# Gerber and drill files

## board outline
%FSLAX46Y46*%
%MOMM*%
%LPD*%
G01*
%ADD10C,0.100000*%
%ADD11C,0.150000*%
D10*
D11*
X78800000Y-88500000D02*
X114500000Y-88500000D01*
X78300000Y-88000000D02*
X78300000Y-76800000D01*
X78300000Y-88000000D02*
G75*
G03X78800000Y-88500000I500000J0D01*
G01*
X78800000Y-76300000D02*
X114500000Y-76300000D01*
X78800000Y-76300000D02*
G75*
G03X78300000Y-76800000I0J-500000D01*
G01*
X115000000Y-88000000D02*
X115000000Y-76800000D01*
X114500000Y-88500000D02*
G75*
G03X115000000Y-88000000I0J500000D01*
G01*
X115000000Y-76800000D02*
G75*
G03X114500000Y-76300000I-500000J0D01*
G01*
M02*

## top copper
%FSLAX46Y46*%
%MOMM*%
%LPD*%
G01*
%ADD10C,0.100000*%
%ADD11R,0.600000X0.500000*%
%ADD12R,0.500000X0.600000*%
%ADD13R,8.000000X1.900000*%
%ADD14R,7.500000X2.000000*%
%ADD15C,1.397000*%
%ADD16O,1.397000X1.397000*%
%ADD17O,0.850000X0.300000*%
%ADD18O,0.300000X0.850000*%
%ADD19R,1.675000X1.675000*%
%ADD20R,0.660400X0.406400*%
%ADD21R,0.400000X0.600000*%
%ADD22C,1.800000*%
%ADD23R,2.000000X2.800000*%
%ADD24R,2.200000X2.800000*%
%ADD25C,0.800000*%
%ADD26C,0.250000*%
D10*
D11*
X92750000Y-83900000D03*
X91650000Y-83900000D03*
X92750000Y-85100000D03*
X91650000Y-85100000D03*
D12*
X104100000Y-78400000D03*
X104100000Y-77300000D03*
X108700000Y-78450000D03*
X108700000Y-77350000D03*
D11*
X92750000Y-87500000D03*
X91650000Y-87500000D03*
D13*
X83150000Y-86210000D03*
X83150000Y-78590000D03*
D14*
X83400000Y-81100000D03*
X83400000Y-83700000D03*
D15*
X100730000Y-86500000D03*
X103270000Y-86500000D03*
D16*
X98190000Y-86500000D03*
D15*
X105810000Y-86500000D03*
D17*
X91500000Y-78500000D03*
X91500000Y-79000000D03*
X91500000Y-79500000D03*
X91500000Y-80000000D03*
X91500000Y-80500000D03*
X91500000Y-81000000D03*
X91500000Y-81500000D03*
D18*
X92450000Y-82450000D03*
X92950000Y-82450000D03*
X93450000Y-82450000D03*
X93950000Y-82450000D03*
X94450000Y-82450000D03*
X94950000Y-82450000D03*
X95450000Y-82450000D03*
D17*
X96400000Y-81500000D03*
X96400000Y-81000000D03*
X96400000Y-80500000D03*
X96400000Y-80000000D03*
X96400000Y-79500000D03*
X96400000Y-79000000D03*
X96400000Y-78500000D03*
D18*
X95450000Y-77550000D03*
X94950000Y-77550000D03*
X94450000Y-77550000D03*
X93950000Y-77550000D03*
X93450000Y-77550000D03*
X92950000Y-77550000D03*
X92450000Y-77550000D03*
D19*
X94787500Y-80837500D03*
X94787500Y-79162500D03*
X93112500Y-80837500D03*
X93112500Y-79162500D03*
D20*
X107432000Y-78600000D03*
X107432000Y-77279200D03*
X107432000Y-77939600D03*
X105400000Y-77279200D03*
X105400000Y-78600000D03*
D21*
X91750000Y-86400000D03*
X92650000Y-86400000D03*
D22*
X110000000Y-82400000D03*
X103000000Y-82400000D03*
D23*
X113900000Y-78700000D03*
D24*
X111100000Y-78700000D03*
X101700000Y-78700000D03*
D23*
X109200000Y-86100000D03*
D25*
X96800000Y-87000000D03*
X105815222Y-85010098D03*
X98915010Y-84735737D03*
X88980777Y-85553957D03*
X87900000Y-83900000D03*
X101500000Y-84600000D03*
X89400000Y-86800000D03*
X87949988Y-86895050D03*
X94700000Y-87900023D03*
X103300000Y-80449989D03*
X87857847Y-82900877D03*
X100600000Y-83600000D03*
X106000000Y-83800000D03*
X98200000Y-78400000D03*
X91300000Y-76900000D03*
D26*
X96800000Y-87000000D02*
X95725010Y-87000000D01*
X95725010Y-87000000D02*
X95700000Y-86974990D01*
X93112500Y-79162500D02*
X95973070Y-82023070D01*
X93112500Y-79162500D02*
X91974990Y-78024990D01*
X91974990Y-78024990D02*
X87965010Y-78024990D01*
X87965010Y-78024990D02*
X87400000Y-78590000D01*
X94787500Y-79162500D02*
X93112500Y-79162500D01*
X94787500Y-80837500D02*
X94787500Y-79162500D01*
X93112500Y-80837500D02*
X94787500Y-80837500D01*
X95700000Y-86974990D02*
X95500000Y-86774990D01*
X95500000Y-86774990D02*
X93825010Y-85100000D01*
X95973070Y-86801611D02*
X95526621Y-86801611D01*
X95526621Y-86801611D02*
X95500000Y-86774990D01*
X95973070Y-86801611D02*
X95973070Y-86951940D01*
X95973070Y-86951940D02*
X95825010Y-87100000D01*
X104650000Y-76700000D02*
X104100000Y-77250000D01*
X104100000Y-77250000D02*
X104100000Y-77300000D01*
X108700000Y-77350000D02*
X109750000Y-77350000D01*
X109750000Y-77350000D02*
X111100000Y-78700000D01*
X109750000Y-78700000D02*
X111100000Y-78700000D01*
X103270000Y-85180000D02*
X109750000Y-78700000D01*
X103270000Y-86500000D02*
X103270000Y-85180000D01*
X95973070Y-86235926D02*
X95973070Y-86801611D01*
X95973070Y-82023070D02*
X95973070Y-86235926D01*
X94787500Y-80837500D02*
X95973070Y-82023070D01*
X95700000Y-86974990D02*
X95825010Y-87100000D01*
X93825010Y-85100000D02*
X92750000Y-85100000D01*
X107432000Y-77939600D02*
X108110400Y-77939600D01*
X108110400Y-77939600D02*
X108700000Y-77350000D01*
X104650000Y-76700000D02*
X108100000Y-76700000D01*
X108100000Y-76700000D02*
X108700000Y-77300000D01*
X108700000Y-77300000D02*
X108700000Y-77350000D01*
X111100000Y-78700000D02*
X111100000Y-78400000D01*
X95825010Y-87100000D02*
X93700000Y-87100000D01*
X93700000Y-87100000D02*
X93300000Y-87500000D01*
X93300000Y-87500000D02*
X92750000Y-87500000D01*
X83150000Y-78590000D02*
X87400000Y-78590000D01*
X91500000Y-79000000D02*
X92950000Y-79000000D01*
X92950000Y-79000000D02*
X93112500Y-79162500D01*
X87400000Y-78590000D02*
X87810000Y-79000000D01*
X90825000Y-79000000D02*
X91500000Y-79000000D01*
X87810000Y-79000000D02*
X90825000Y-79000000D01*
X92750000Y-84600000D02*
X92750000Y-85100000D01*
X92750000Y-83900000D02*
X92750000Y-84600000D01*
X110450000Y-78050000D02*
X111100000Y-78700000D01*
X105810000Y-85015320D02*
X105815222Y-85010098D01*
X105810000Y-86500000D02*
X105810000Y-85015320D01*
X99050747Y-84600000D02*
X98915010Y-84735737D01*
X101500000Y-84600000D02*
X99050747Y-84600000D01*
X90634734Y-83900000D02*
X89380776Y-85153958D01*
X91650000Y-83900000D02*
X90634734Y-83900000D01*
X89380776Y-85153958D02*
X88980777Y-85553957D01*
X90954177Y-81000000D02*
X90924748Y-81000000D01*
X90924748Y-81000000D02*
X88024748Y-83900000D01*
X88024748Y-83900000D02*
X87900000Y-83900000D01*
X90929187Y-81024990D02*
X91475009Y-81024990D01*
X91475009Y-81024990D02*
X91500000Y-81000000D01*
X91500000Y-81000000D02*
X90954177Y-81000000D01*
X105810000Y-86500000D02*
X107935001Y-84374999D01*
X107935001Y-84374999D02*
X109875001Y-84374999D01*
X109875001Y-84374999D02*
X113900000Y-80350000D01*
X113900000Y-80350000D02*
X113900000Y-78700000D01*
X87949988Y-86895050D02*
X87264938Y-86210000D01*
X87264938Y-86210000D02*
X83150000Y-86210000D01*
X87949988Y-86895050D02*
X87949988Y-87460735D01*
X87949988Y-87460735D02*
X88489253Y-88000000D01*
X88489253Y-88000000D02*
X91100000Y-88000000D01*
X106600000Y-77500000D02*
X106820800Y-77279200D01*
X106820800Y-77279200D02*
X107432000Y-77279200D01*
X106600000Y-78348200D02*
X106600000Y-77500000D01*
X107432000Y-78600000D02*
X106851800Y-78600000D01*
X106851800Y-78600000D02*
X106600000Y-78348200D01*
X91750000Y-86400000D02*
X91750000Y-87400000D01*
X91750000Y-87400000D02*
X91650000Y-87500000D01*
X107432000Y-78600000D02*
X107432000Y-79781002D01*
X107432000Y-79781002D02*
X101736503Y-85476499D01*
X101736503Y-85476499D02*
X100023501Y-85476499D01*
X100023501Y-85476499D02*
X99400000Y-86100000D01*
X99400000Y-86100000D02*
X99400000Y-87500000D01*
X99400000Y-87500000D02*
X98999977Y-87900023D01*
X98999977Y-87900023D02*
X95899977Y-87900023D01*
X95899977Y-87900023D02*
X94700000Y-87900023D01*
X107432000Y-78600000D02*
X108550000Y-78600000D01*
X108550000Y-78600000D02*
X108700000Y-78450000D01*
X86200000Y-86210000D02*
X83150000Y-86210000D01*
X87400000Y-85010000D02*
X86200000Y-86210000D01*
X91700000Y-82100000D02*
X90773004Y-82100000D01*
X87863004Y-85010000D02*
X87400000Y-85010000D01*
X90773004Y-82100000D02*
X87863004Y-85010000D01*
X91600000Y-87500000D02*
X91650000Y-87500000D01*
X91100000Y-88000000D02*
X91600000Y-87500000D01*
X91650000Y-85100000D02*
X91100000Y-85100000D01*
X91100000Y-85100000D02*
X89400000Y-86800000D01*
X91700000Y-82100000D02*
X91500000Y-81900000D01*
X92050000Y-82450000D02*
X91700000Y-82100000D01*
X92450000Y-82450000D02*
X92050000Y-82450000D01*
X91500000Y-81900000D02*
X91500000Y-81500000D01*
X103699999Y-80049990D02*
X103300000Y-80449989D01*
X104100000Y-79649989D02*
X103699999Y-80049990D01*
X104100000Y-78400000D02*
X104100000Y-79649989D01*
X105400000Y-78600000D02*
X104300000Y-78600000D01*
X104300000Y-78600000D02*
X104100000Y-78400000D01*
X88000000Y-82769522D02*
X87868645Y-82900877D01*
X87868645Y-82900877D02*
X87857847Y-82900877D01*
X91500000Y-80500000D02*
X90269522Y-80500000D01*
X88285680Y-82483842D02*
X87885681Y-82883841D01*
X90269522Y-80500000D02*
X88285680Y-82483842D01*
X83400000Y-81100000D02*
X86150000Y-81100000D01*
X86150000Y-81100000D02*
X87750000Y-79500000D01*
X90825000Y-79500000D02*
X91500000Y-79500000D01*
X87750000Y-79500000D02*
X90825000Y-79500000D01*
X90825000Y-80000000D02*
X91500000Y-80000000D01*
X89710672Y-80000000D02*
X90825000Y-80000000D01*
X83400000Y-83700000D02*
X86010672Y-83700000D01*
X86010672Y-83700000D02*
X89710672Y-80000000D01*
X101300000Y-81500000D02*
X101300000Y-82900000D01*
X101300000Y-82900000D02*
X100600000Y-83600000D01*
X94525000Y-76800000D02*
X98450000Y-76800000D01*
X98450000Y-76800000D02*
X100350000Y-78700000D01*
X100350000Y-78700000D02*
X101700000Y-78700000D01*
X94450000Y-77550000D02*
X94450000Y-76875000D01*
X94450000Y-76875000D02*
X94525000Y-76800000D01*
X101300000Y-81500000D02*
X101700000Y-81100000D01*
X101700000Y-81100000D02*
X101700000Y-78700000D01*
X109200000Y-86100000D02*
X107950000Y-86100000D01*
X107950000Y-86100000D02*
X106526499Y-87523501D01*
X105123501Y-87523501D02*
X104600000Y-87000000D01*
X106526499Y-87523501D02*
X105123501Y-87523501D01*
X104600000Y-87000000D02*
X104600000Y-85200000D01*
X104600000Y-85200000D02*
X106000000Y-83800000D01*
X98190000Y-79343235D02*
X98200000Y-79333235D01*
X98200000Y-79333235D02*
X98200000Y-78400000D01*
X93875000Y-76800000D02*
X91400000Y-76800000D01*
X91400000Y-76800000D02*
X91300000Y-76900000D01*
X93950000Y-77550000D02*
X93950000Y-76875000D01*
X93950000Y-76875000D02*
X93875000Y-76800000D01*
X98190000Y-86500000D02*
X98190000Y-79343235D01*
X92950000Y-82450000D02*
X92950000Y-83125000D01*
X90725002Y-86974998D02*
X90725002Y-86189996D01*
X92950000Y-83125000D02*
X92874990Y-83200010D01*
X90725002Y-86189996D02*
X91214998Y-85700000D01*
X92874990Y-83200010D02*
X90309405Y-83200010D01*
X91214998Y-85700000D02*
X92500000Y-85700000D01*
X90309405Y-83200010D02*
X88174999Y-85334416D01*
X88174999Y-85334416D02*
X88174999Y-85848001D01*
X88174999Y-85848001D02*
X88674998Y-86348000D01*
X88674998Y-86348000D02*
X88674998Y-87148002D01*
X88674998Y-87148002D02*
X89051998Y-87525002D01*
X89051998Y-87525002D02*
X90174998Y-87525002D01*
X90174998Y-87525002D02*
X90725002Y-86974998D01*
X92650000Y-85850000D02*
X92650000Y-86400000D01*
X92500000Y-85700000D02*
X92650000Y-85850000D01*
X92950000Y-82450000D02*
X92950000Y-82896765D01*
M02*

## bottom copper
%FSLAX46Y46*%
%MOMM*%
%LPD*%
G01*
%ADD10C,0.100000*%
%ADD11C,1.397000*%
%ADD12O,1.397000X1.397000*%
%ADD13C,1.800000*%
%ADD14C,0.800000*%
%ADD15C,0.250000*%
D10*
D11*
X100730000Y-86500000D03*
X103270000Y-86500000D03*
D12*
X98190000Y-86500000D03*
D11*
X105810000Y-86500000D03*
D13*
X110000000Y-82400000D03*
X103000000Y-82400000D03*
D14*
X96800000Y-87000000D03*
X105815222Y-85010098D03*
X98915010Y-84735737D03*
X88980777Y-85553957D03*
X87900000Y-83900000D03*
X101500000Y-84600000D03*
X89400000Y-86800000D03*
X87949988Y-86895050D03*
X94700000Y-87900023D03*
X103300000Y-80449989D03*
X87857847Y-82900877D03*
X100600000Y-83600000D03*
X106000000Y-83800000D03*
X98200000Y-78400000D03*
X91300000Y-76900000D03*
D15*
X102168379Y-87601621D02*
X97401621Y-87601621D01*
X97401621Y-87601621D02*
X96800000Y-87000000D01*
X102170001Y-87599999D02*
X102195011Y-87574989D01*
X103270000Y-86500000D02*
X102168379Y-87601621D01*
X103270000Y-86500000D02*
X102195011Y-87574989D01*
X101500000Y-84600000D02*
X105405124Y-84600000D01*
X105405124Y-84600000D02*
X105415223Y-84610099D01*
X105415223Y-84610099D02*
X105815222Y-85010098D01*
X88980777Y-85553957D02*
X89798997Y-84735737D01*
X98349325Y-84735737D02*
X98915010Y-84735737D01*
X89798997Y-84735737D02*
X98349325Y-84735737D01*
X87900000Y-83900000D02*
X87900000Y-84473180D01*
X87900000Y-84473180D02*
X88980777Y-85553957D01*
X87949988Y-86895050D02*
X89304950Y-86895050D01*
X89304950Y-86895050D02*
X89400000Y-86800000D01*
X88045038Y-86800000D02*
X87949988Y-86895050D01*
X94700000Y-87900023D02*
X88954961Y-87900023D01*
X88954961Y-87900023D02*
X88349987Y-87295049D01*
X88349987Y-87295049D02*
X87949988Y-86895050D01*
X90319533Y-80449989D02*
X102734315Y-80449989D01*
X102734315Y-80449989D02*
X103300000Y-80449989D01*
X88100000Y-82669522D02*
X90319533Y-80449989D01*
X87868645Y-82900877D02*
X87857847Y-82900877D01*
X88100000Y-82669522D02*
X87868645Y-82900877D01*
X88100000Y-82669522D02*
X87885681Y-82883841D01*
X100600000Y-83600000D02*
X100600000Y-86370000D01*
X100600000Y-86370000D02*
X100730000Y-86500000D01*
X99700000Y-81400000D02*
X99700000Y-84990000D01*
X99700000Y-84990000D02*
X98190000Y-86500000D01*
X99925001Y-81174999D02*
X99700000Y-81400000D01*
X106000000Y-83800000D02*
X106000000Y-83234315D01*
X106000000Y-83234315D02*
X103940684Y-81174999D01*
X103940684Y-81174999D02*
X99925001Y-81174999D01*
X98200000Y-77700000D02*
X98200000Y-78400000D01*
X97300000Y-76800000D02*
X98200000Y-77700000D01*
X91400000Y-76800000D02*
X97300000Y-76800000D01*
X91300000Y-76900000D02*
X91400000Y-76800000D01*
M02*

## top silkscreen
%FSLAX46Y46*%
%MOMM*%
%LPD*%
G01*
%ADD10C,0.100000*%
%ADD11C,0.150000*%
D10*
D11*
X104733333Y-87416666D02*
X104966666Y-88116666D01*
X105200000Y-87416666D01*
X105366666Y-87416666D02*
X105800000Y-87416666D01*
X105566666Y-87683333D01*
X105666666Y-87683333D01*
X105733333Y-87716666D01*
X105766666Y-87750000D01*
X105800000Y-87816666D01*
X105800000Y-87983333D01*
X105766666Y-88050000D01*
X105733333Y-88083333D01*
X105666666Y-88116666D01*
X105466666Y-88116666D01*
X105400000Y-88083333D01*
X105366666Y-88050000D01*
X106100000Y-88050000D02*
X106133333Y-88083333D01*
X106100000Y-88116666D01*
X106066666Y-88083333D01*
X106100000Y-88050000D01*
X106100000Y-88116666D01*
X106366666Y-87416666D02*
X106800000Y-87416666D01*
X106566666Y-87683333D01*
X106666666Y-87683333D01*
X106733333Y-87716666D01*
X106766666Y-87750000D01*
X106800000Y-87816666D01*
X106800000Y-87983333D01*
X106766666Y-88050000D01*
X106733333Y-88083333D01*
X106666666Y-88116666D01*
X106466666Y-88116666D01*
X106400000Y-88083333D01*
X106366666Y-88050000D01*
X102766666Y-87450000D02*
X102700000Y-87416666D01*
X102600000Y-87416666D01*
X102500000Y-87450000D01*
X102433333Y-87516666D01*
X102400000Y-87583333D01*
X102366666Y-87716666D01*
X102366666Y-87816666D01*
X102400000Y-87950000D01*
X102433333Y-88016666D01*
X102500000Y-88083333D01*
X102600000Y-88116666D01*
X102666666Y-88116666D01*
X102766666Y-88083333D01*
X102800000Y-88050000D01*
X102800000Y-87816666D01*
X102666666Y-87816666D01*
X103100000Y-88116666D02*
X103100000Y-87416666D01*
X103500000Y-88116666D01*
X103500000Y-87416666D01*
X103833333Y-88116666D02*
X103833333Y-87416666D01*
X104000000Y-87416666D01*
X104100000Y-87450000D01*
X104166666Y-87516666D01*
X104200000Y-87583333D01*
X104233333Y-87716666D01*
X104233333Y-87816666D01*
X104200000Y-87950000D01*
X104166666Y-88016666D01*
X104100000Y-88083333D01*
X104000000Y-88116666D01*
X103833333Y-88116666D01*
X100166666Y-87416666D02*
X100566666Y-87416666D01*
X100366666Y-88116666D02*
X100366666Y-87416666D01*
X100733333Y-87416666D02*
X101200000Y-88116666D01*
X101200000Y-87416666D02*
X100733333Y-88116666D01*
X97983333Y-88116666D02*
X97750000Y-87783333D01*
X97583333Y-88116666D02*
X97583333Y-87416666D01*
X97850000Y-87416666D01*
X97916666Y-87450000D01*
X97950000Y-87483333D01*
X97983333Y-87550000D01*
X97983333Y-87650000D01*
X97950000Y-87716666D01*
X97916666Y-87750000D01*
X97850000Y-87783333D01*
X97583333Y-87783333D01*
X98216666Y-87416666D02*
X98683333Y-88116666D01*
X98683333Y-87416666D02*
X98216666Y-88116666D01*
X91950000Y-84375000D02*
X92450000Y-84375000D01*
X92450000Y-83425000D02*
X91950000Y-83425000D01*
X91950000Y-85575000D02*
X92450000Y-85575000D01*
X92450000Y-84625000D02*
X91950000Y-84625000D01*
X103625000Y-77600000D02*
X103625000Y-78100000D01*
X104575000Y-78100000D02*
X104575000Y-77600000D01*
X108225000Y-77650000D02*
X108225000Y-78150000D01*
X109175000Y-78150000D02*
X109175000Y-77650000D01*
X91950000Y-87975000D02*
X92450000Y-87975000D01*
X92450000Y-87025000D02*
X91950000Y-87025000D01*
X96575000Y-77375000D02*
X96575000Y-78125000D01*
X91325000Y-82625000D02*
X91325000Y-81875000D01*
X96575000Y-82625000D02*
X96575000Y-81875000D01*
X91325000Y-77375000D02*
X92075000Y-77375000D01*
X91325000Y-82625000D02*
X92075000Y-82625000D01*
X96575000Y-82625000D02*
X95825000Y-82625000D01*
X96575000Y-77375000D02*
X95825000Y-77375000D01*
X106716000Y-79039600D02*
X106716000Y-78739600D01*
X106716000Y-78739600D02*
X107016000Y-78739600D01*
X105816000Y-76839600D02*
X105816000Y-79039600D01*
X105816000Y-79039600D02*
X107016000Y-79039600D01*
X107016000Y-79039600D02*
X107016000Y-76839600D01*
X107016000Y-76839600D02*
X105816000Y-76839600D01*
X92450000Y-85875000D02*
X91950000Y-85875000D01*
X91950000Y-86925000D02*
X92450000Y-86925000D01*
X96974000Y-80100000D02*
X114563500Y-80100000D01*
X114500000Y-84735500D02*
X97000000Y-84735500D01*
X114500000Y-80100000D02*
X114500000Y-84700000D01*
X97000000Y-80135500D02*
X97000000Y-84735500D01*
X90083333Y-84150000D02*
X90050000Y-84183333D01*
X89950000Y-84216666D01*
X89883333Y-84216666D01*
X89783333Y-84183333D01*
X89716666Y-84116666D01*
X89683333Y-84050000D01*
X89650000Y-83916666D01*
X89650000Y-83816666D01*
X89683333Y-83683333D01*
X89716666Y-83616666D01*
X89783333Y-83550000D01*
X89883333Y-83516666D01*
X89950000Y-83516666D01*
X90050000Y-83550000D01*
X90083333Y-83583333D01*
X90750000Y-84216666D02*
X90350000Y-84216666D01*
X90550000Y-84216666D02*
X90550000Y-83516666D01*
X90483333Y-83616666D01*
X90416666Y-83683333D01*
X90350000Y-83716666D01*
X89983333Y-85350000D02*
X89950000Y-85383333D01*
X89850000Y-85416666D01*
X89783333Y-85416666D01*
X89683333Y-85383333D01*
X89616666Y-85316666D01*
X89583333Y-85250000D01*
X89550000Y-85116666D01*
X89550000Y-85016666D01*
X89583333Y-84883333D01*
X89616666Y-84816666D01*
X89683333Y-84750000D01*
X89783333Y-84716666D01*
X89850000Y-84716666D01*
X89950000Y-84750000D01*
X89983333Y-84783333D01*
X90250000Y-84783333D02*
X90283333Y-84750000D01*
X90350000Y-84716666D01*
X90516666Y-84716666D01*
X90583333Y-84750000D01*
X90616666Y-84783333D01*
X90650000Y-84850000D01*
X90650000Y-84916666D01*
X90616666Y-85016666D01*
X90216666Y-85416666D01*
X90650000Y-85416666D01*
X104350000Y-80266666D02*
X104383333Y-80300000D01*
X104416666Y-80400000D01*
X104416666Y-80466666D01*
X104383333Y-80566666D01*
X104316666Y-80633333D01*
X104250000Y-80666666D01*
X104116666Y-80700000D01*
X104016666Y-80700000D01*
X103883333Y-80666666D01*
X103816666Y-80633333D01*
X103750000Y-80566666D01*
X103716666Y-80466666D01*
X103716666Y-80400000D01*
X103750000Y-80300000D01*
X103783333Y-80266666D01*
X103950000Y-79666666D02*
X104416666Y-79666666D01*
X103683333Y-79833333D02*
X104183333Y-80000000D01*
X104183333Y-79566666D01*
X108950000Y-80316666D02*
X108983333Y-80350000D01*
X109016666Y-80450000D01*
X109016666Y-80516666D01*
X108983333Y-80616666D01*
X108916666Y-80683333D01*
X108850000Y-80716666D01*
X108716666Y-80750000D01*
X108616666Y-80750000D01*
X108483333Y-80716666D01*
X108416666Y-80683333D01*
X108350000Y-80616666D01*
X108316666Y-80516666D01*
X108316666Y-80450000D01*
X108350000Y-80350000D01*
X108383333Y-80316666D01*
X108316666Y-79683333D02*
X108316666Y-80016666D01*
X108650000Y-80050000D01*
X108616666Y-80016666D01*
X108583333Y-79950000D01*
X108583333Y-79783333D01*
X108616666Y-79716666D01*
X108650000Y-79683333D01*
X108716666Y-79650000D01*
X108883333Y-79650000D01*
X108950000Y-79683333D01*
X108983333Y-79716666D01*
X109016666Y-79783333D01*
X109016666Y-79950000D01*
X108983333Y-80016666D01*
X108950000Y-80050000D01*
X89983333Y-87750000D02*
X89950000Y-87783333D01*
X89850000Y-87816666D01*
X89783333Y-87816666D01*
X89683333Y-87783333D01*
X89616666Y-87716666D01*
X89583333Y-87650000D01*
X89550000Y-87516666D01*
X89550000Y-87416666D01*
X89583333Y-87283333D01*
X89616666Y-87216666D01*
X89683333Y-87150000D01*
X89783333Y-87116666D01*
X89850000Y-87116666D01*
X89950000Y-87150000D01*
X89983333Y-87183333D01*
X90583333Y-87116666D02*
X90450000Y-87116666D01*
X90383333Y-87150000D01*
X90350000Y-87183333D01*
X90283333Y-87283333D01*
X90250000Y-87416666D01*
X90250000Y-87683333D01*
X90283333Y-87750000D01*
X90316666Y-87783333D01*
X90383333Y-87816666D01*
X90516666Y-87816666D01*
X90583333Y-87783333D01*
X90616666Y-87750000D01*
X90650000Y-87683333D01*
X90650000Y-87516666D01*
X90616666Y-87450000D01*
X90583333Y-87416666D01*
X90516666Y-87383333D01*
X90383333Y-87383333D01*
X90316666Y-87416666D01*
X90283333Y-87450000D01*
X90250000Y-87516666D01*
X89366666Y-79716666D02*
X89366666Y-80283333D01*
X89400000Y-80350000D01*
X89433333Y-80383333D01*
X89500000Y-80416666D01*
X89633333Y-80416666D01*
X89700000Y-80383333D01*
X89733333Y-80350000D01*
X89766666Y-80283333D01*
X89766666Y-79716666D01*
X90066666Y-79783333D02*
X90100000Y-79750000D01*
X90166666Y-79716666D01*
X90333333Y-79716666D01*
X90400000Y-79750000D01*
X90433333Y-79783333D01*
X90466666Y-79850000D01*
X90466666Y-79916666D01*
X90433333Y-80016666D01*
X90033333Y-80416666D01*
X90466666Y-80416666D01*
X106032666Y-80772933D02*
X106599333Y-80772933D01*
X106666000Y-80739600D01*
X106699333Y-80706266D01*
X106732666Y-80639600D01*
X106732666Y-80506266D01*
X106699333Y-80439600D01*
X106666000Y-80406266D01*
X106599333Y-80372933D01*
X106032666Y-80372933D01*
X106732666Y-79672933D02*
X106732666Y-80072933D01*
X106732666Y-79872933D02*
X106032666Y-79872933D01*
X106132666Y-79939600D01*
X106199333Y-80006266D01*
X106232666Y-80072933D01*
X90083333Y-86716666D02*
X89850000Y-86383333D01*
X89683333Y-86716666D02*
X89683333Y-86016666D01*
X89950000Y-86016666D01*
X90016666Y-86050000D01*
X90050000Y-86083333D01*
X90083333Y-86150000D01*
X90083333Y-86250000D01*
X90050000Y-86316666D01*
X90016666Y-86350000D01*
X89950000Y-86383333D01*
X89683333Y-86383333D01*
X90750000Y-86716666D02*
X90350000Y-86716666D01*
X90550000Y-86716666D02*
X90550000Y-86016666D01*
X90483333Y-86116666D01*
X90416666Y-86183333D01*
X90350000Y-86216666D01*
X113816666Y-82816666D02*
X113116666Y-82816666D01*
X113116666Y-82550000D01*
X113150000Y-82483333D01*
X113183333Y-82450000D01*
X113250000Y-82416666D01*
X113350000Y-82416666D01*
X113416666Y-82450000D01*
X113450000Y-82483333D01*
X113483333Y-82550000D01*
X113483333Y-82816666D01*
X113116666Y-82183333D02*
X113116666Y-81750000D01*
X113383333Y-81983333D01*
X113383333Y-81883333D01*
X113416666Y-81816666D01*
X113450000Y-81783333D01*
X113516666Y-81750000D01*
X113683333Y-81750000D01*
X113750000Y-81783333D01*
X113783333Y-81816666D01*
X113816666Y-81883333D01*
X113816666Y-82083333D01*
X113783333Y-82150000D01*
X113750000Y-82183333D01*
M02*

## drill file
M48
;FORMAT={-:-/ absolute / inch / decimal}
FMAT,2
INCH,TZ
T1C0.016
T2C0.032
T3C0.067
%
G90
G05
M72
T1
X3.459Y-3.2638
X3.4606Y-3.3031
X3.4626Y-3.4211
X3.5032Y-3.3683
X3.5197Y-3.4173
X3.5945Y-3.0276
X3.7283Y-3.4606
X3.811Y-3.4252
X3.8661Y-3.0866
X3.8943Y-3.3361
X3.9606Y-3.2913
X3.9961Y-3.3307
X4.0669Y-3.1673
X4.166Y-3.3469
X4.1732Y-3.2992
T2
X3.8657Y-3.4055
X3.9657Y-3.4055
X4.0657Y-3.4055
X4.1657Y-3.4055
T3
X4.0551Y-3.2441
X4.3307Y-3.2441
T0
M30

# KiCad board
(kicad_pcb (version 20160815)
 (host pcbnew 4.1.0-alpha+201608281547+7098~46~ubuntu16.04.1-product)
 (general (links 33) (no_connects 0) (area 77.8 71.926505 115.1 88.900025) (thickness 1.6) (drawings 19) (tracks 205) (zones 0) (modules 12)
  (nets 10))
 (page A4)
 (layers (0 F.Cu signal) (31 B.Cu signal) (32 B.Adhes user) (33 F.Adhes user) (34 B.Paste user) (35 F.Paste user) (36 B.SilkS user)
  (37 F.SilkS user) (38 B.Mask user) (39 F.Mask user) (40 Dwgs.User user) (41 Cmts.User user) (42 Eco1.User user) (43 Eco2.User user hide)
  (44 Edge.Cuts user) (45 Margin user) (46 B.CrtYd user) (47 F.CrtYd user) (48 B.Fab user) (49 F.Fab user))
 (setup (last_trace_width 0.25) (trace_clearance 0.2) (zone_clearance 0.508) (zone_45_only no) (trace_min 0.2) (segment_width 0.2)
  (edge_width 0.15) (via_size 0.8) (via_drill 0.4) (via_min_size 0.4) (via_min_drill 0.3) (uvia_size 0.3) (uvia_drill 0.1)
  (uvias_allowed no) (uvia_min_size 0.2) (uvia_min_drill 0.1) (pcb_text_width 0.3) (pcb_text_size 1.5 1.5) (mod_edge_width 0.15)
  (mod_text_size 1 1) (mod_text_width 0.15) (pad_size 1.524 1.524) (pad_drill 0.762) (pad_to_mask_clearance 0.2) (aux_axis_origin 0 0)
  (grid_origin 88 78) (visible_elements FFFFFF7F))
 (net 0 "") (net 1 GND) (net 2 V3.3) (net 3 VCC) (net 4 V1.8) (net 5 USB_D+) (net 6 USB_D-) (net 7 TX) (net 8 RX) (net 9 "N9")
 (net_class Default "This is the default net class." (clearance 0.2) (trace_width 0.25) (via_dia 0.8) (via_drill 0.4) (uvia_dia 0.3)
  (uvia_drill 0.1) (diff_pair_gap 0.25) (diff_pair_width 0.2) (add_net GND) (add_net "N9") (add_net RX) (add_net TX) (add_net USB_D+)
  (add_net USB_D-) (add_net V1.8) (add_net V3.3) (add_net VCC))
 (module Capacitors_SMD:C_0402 (layer F.Cu) (at 92.2 83.9 180)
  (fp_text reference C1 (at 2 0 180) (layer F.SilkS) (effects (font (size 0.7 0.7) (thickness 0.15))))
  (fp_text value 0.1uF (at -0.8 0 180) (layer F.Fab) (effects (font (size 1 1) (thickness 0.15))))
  (fp_line (start 0.25 -0.475) (end -0.25 -0.475) (layer F.SilkS) (width 0.15))
  (fp_line (start -0.25 0.475) (end 0.25 0.475) (layer F.SilkS) (width 0.15))
  (pad 1 smd rect (at -0.55 0 180) (size 0.6 0.5) (layers F.Cu F.Paste F.Mask) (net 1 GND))
  (pad 2 smd rect (at 0.55 0 180) (size 0.6 0.5) (layers F.Cu F.Paste F.Mask) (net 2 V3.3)))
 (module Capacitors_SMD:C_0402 (layer F.Cu) (at 92.2 85.1 180)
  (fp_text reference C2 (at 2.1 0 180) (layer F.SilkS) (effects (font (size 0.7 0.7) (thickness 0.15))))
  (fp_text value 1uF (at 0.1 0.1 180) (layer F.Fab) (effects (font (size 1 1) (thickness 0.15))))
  (fp_line (start 0.25 -0.475) (end -0.25 -0.475) (layer F.SilkS) (width 0.15))
  (fp_line (start -0.25 0.475) (end 0.25 0.475) (layer F.SilkS) (width 0.15))
  (pad 1 smd rect (at -0.55 0 180) (size 0.6 0.5) (layers F.Cu F.Paste F.Mask) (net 1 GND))
  (pad 2 smd rect (at 0.55 0 180) (size 0.6 0.5) (layers F.Cu F.Paste F.Mask) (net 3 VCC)))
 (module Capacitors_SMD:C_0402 (layer F.Cu) (at 104.1 77.85 90)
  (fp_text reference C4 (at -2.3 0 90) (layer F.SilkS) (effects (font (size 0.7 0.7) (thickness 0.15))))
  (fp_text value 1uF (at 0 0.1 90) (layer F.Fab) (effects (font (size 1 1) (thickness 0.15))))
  (fp_line (start 0.25 -0.475) (end -0.25 -0.475) (layer F.SilkS) (width 0.15))
  (fp_line (start -0.25 0.475) (end 0.25 0.475) (layer F.SilkS) (width 0.15))
  (pad 1 smd rect (at -0.55 0 90) (size 0.6 0.5) (layers F.Cu F.Paste F.Mask) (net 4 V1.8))
  (pad 2 smd rect (at 0.55 0 90) (size 0.6 0.5) (layers F.Cu F.Paste F.Mask) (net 1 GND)))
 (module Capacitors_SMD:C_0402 (layer F.Cu) (at 108.7 77.9 90)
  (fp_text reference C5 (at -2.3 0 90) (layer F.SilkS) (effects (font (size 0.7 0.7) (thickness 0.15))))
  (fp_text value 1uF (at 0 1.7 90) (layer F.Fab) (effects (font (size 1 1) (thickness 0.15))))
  (fp_line (start 0.25 -0.475) (end -0.25 -0.475) (layer F.SilkS) (width 0.15))
  (fp_line (start -0.25 0.475) (end 0.25 0.475) (layer F.SilkS) (width 0.15))
  (pad 1 smd rect (at -0.55 0 90) (size 0.6 0.5) (layers F.Cu F.Paste F.Mask) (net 3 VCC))
  (pad 2 smd rect (at 0.55 0 90) (size 0.6 0.5) (layers F.Cu F.Paste F.Mask) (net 1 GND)))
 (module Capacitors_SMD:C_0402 (layer F.Cu) (at 92.2 87.5 180)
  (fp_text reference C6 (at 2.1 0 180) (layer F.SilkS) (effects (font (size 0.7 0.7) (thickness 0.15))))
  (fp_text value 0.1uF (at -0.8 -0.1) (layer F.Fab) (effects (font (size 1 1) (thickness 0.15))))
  (fp_line (start 0.25 -0.475) (end -0.25 -0.475) (layer F.SilkS) (width 0.15))
  (fp_line (start -0.25 0.475) (end 0.25 0.475) (layer F.SilkS) (width 0.15))
  (pad 1 smd rect (at -0.55 0 180) (size 0.6 0.5) (layers F.Cu F.Paste F.Mask) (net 1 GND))
  (pad 2 smd rect (at 0.55 0 180) (size 0.6 0.5) (layers F.Cu F.Paste F.Mask) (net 3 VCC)))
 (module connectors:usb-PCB (layer F.Cu) (at 78.25 82.4 270)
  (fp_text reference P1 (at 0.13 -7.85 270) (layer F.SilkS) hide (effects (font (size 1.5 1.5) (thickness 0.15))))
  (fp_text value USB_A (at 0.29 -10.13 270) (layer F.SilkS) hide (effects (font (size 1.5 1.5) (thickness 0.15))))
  (pad 1 connect rect (at 3.81 -4.9 270) (size 1.9 8) (layers F.Cu F.Mask) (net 3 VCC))
  (pad 4 connect rect (at -3.81 -4.9 270) (size 1.9 8) (layers F.Cu F.Mask) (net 1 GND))
  (pad 3 connect rect (at -1.3 -5.15 270) (size 2 7.5) (layers F.Cu F.Mask) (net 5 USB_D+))
  (pad 2 connect rect (at 1.3 -5.15 270) (size 2 7.5) (layers F.Cu F.Mask) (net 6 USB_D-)))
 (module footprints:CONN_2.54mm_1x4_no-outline (layer F.Cu) (at 102 86.5 180)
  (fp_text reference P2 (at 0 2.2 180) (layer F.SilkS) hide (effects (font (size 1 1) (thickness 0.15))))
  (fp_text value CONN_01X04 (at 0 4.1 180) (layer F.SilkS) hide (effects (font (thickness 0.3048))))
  (pad 2 thru_hole circle (at 1.27 0 180) (size 1.397 1.397) (drill 0.8128) (layers *.Cu *.Mask F.SilkS) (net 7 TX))
  (pad 3 thru_hole circle (at -1.27 0 180) (size 1.397 1.397) (drill 0.8128) (layers *.Cu *.Mask F.SilkS) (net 1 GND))
  (pad 1 thru_hole oval (at 3.81 0 180) (size 1.397 1.397) (drill 0.8128) (layers *.Cu *.Mask F.SilkS) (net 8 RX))
  (pad 4 thru_hole circle (at -3.81 0 180) (size 1.397 1.397) (drill 0.8128) (layers *.Cu *.Mask F.SilkS) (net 2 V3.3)))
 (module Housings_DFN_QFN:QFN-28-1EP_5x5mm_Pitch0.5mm (layer F.Cu) (at 93.95 80)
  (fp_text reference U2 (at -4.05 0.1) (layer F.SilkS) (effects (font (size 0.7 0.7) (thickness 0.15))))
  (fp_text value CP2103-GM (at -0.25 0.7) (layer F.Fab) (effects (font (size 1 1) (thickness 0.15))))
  (fp_line (start 2.625 -2.625) (end 2.625 -1.875) (layer F.SilkS) (width 0.15))
  (fp_line (start -2.625 2.625) (end -2.625 1.875) (layer F.SilkS) (width 0.15))
  (fp_line (start 2.625 2.625) (end 2.625 1.875) (layer F.SilkS) (width 0.15))
  (fp_line (start -2.625 -2.625) (end -1.875 -2.625) (layer F.SilkS) (width 0.15))
  (fp_line (start -2.625 2.625) (end -1.875 2.625) (layer F.SilkS) (width 0.15))
  (fp_line (start 2.625 2.625) (end 1.875 2.625) (layer F.SilkS) (width 0.15))
  (fp_line (start 2.625 -2.625) (end 1.875 -2.625) (layer F.SilkS) (width 0.15))
  (pad 1 smd oval (at -2.45 -1.5) (size 0.85 0.3) (layers F.Cu F.Paste F.Mask))
  (pad 2 smd oval (at -2.45 -1) (size 0.85 0.3) (layers F.Cu F.Paste F.Mask) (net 1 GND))
  (pad 3 smd oval (at -2.45 -0.5) (size 0.85 0.3) (layers F.Cu F.Paste F.Mask) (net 5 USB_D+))
  (pad 4 smd oval (at -2.45 0) (size 0.85 0.3) (layers F.Cu F.Paste F.Mask) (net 6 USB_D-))
  (pad 5 smd oval (at -2.45 0.5) (size 0.85 0.3) (layers F.Cu F.Paste F.Mask) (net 4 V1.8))
  (pad 6 smd oval (at -2.45 1) (size 0.85 0.3) (layers F.Cu F.Paste F.Mask) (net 2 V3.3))
  (pad 7 smd oval (at -2.45 1.5) (size 0.85 0.3) (layers F.Cu F.Paste F.Mask) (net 3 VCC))
  (pad 8 smd oval (at -1.5 2.45 90) (size 0.85 0.3) (layers F.Cu F.Paste F.Mask) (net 3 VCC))
  (pad 9 smd oval (at -1 2.45 90) (size 0.85 0.3) (layers F.Cu F.Paste F.Mask) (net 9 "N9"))
  (pad 10 smd oval (at -0.5 2.45 90) (size 0.85 0.3) (layers F.Cu F.Paste F.Mask))
  (pad 11 smd oval (at 0 2.45 90) (size 0.85 0.3) (layers F.Cu F.Paste F.Mask))
  (pad 12 smd oval (at 0.5 2.45 90) (size 0.85 0.3) (layers F.Cu F.Paste F.Mask))
  (pad 13 smd oval (at 1 2.45 90) (size 0.85 0.3) (layers F.Cu F.Paste F.Mask))
  (pad 14 smd oval (at 1.5 2.45 90) (size 0.85 0.3) (layers F.Cu F.Paste F.Mask))
  (pad 15 smd oval (at 2.45 1.5) (size 0.85 0.3) (layers F.Cu F.Paste F.Mask))
  (pad 16 smd oval (at 2.45 1) (size 0.85 0.3) (layers F.Cu F.Paste F.Mask))
  (pad 17 smd oval (at 2.45 0.5) (size 0.85 0.3) (layers F.Cu F.Paste F.Mask))
  (pad 18 smd oval (at 2.45 0) (size 0.85 0.3) (layers F.Cu F.Paste F.Mask))
  (pad 19 smd oval (at 2.45 -0.5) (size 0.85 0.3) (layers F.Cu F.Paste F.Mask))
  (pad 20 smd oval (at 2.45 -1) (size 0.85 0.3) (layers F.Cu F.Paste F.Mask))
  (pad 21 smd oval (at 2.45 -1.5) (size 0.85 0.3) (layers F.Cu F.Paste F.Mask))
  (pad 22 smd oval (at 1.5 -2.45 90) (size 0.85 0.3) (layers F.Cu F.Paste F.Mask))
  (pad 23 smd oval (at 1 -2.45 90) (size 0.85 0.3) (layers F.Cu F.Paste F.Mask))
  (pad 24 smd oval (at 0.5 -2.45 90) (size 0.85 0.3) (layers F.Cu F.Paste F.Mask) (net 7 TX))
  (pad 25 smd oval (at 0 -2.45 90) (size 0.85 0.3) (layers F.Cu F.Paste F.Mask) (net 8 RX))
  (pad 26 smd oval (at -0.5 -2.45 90) (size 0.85 0.3) (layers F.Cu F.Paste F.Mask))
  (pad 27 smd oval (at -1 -2.45 90) (size 0.85 0.3) (layers F.Cu F.Paste F.Mask))
  (pad 28 smd oval (at -1.5 -2.45 90) (size 0.85 0.3) (layers F.Cu F.Paste F.Mask))
  (pad 29 smd rect (at 0.8375 0.8375) (size 1.675 1.675) (layers F.Cu F.Paste F.Mask) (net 1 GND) (solder_paste_margin_ratio -0.2))
  (pad 29 smd rect (at 0.8375 -0.8375) (size 1.675 1.675) (layers F.Cu F.Paste F.Mask) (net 1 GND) (solder_paste_margin_ratio -0.2))
  (pad 29 smd rect (at -0.8375 0.8375) (size 1.675 1.675) (layers F.Cu F.Paste F.Mask) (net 1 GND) (solder_paste_margin_ratio -0.2))
  (pad 29 smd rect (at -0.8375 -0.8375) (size 1.675 1.675) (layers F.Cu F.Paste F.Mask) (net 1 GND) (solder_paste_margin_ratio -0.2)))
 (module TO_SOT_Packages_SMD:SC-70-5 (layer F.Cu) (at 106.416 77.9396 90)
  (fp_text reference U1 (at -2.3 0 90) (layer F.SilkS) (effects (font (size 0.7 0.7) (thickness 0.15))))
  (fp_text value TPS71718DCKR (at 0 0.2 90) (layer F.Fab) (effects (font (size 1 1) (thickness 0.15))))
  (fp_line (start -1.1 0.3) (end -0.8 0.3) (layer F.SilkS) (width 0.15))
  (fp_line (start -0.8 0.3) (end -0.8 0.6) (layer F.SilkS) (width 0.15))
  (fp_line (start 1.1 -0.6) (end -1.1 -0.6) (layer F.SilkS) (width 0.15))
  (fp_line (start -1.1 -0.6) (end -1.1 0.6) (layer F.SilkS) (width 0.15))
  (fp_line (start -1.1 0.6) (end 1.1 0.6) (layer F.SilkS) (width 0.15))
  (fp_line (start 1.1 0.6) (end 1.1 -0.6) (layer F.SilkS) (width 0.15))
  (pad 1 smd rect (at -0.6604 1.016 90) (size 0.4064 0.6604) (layers F.Cu F.Paste F.Mask) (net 3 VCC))
  (pad 3 smd rect (at 0.6604 1.016 90) (size 0.4064 0.6604) (layers F.Cu F.Paste F.Mask) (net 3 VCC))
  (pad 2 smd rect (at 0 1.016 90) (size 0.4064 0.6604) (layers F.Cu F.Paste F.Mask) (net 1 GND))
  (pad 4 smd rect (at 0.6604 -1.016 90) (size 0.4064 0.6604) (layers F.Cu F.Paste F.Mask))
  (pad 5 smd rect (at -0.6604 -1.016 90) (size 0.4064 0.6604) (layers F.Cu F.Paste F.Mask) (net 4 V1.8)))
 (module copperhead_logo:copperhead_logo (layer B.Cu) (at 94.2 82.1)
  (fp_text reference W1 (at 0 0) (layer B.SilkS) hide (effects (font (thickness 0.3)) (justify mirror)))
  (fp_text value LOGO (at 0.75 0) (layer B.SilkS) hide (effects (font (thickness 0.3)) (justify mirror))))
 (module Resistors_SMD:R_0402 (layer F.Cu) (at 92.2 86.4)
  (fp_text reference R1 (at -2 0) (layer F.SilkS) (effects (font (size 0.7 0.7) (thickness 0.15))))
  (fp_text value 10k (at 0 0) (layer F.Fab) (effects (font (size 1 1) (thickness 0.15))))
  (fp_line (start 0.25 -0.525) (end -0.25 -0.525) (layer F.SilkS) (width 0.15))
  (fp_line (start -0.25 0.525) (end 0.25 0.525) (layer F.SilkS) (width 0.15))
  (pad 1 smd rect (at -0.45 0) (size 0.4 0.6) (layers F.Cu F.Paste F.Mask) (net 3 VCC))
  (pad 2 smd rect (at 0.45 0) (size 0.4 0.6) (layers F.Cu F.Paste F.Mask) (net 9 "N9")))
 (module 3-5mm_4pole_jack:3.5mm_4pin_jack (layer F.Cu) (at 114.5 80.1 270)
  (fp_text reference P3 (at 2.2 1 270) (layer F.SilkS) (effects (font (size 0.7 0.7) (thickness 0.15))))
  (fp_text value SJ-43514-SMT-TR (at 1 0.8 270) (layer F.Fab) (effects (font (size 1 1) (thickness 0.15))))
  (fp_line (start 0 17.526) (end 0 -0.0635) (layer F.SilkS) (width 0.15))
  (fp_line (start 4.6355 0) (end 4.6355 17.5) (layer F.SilkS) (width 0.15))
  (fp_line (start 0 0) (end 4.6 0) (layer F.SilkS) (width 0.15))
  (fp_line (start 0.0355 17.5) (end 4.6355 17.5) (layer F.SilkS) (width 0.15))
  (pad "" np_thru_hole circle (at 2.3 4.5 270) (size 1.8 1.8) (drill 1.7) (layers *.Cu *.Mask))
  (pad "" np_thru_hole circle (at 2.3 11.5 270) (size 1.8 1.8) (drill 1.7) (layers *.Cu *.Mask))
  (pad 1 smd rect (at -1.4 0.6 270) (size 2.8 2) (layers F.Cu F.Paste F.Mask) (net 2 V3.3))
  (pad 4 smd rect (at -1.4 3.4 270) (size 2.8 2.2) (layers F.Cu F.Paste F.Mask) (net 1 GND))
  (pad 2 smd rect (at -1.4 12.8 270) (size 2.8 2.2) (layers F.Cu F.Paste F.Mask) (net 7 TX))
  (pad 3 smd rect (at 6 5.3 270) (size 2.8 2) (layers F.Cu F.Paste F.Mask) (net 8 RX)))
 (gr_line (start 78.8 88.5) (end 114.5 88.5) (layer Edge.Cuts) (width 0.15))
 (gr_line (start 78.3 88) (end 78.3 76.8) (layer Edge.Cuts) (width 0.15))
 (gr_arc (start 78.8 88) (end 78.8 88.5) (angle 90) (layer Edge.Cuts) (width 0.15))
 (gr_line (start 78.8 76.3) (end 114.5 76.3) (layer Edge.Cuts) (width 0.15))
 (gr_arc (start 78.8 76.8) (end 78.3 76.8) (angle 90) (layer Edge.Cuts) (width 0.15))
 (gr_line (start 115 88) (end 115 76.8) (layer Edge.Cuts) (width 0.15))
 (gr_arc (start 114.5 88) (end 115 88) (angle 90) (layer Edge.Cuts) (width 0.15))
 (gr_arc (start 114.5 76.8) (end 114.5 76.3) (angle 90) (layer Edge.Cuts) (width 0.15))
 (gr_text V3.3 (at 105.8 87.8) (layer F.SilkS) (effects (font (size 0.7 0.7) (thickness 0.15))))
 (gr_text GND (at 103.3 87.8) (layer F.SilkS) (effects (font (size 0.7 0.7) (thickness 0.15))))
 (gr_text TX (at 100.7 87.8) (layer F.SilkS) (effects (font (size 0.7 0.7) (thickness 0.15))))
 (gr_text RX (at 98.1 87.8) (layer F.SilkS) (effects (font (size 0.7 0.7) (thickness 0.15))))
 (segment (start 102.168379 87.601621) (end 97.401621 87.601621) (width 0.25) (layer B.Cu) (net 1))
 (segment (start 97.401621 87.601621) (end 96.8 87) (width 0.25) (layer B.Cu) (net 1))
 (segment (start 96.8 87) (end 95.72501 87) (width 0.25) (layer F.Cu) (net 1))
 (segment (start 95.72501 87) (end 95.7 86.97499) (width 0.25) (layer F.Cu) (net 1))
 (segment (start 102.170001 87.599999) (end 102.195011 87.574989) (width 0.25) (layer B.Cu) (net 1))
 (segment (start 93.1125 79.1625) (end 95.97307 82.02307) (width 0.25) (layer F.Cu) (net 1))
 (segment (start 93.1125 79.1625) (end 91.97499 78.02499) (width 0.25) (layer F.Cu) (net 1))
 (segment (start 91.97499 78.02499) (end 87.96501 78.02499) (width 0.25) (layer F.Cu) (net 1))
 (segment (start 87.96501 78.02499) (end 87.4 78.59) (width 0.25) (layer F.Cu) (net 1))
 (segment (start 94.7875 79.1625) (end 93.1125 79.1625) (width 0.25) (layer F.Cu) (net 1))
 (segment (start 94.7875 80.8375) (end 94.7875 79.1625) (width 0.25) (layer F.Cu) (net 1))
 (segment (start 93.1125 80.8375) (end 94.7875 80.8375) (width 0.25) (layer F.Cu) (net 1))
 (segment (start 95.7 86.97499) (end 95.5 86.77499) (width 0.25) (layer F.Cu) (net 1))
 (segment (start 95.5 86.77499) (end 93.82501 85.1) (width 0.25) (layer F.Cu) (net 1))
 (segment (start 95.97307 86.801611) (end 95.526621 86.801611) (width 0.25) (layer F.Cu) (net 1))
 (segment (start 95.526621 86.801611) (end 95.5 86.77499) (width 0.25) (layer F.Cu) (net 1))
 (segment (start 95.97307 86.801611) (end 95.97307 86.95194) (width 0.25) (layer F.Cu) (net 1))
 (segment (start 95.97307 86.95194) (end 95.82501 87.1) (width 0.25) (layer F.Cu) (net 1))
 (segment (start 104.65 76.7) (end 104.1 77.25) (width 0.25) (layer F.Cu) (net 1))
 (segment (start 104.1 77.25) (end 104.1 77.3) (width 0.25) (layer F.Cu) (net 1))
 (segment (start 108.7 77.35) (end 109.75 77.35) (width 0.25) (layer F.Cu) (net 1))
 (segment (start 109.75 77.35) (end 111.1 78.7) (width 0.25) (layer F.Cu) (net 1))
 (segment (start 109.75 78.7) (end 111.1 78.7) (width 0.25) (layer F.Cu) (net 1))
 (segment (start 103.27 85.18) (end 109.75 78.7) (width 0.25) (layer F.Cu) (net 1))
 (segment (start 103.27 86.5) (end 103.27 85.18) (width 0.25) (layer F.Cu) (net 1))
 (segment (start 95.97307 86.235926) (end 95.97307 86.801611) (width 0.25) (layer F.Cu) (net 1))
 (segment (start 95.97307 82.02307) (end 95.97307 86.235926) (width 0.25) (layer F.Cu) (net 1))
 (segment (start 94.7875 80.8375) (end 95.97307 82.02307) (width 0.25) (layer F.Cu) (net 1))
 (segment (start 103.27 86.5) (end 102.168379 87.601621) (width 0.25) (layer B.Cu) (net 1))
 (via (at 96.8 87) (size 0.8) (drill 0.4) (layers F.Cu B.Cu) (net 1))
 (segment (start 95.7 86.97499) (end 95.82501 87.1) (width 0.25) (layer F.Cu) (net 1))
 (segment (start 93.82501 85.1) (end 92.75 85.1) (width 0.25) (layer F.Cu) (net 1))
 (segment (start 107.432 77.9396) (end 108.1104 77.9396) (width 0.25) (layer F.Cu) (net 1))
 (segment (start 108.1104 77.9396) (end 108.7 77.35) (width 0.25) (layer F.Cu) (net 1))
 (segment (start 104.65 76.7) (end 108.1 76.7) (width 0.25) (layer F.Cu) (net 1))
 (segment (start 108.1 76.7) (end 108.7 77.3) (width 0.25) (layer F.Cu) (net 1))
 (segment (start 108.7 77.3) (end 108.7 77.35) (width 0.25) (layer F.Cu) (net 1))
 (segment (start 111.1 78.7) (end 111.1 78.4) (width 0.25) (layer F.Cu) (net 1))
 (segment (start 95.82501 87.1) (end 93.7 87.1) (width 0.25) (layer F.Cu) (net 1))
 (segment (start 93.7 87.1) (end 93.3 87.5) (width 0.25) (layer F.Cu) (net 1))
 (segment (start 93.3 87.5) (end 92.75 87.5) (width 0.25) (layer F.Cu) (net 1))
 (segment (start 83.15 78.59) (end 87.4 78.59) (width 0.25) (layer F.Cu) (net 1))
 (segment (start 103.27 86.5) (end 102.195011 87.574989) (width 0.25) (layer B.Cu) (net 1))
 (segment (start 91.5 79) (end 92.95 79) (width 0.25) (layer F.Cu) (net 1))
 (segment (start 92.95 79) (end 93.1125 79.1625) (width 0.25) (layer F.Cu) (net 1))
 (segment (start 87.4 78.59) (end 87.81 79) (width 0.25) (layer F.Cu) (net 1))
 (segment (start 90.825 79) (end 91.5 79) (width 0.25) (layer F.Cu) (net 1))
 (segment (start 87.81 79) (end 90.825 79) (width 0.25) (layer F.Cu) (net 1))
 (segment (start 92.75 84.6) (end 92.75 85.1) (width 0.25) (layer F.Cu) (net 1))
 (segment (start 92.75 83.9) (end 92.75 84.6) (width 0.25) (layer F.Cu) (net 1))
 (segment (start 110.45 78.05) (end 111.1 78.7) (width 0.25) (layer F.Cu) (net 1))
 (segment (start 101.5 84.6) (end 105.405124 84.6) (width 0.25) (layer B.Cu) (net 2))
 (segment (start 105.81 85.01532) (end 105.815222 85.010098) (width 0.25) (layer F.Cu) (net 2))
 (segment (start 105.81 86.5) (end 105.81 85.01532) (width 0.25) (layer F.Cu) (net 2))
 (segment (start 105.405124 84.6) (end 105.415223 84.610099) (width 0.25) (layer B.Cu) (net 2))
 (via (at 105.815222 85.010098) (size 0.8) (drill 0.4) (layers F.Cu B.Cu) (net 2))
 (segment (start 105.415223 84.610099) (end 105.815222 85.010098) (width 0.25) (layer B.Cu) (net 2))
 (segment (start 88.980777 85.553957) (end 89.798997 84.735737) (width 0.25) (layer B.Cu) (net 2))
 (segment (start 99.050747 84.6) (end 98.91501 84.735737) (width 0.25) (layer F.Cu) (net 2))
 (segment (start 98.349325 84.735737) (end 98.91501 84.735737) (width 0.25) (layer B.Cu) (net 2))
 (segment (start 89.798997 84.735737) (end 98.349325 84.735737) (width 0.25) (layer B.Cu) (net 2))
 (segment (start 101.5 84.6) (end 99.050747 84.6) (width 0.25) (layer F.Cu) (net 2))
 (via (at 98.91501 84.735737) (size 0.8) (drill 0.4) (layers F.Cu B.Cu) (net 2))
 (segment (start 87.9 83.9) (end 87.9 84.47318) (width 0.25) (layer B.Cu) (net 2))
 (segment (start 87.9 84.47318) (end 88.980777 85.553957) (width 0.25) (layer B.Cu) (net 2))
 (via (at 88.980777 85.553957) (size 0.8) (drill 0.4) (layers F.Cu B.Cu) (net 2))
 (segment (start 90.634734 83.9) (end 89.380776 85.153958) (width 0.25) (layer F.Cu) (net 2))
 (segment (start 91.65 83.9) (end 90.634734 83.9) (width 0.25) (layer F.Cu) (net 2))
 (segment (start 89.380776 85.153958) (end 88.980777 85.553957) (width 0.25) (layer F.Cu) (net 2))
 (segment (start 90.954177 81) (end 90.924748 81) (width 0.25) (layer F.Cu) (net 2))
 (segment (start 90.924748 81) (end 88.024748 83.9) (width 0.25) (layer F.Cu) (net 2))
 (segment (start 88.024748 83.9) (end 87.9 83.9) (width 0.25) (layer F.Cu) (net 2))
 (via (at 87.9 83.9) (size 0.8) (drill 0.4) (layers F.Cu B.Cu) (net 2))
 (segment (start 90.929187 81.02499) (end 91.475009 81.02499) (width 0.25) (layer F.Cu) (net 2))
 (segment (start 91.475009 81.02499) (end 91.5 81) (width 0.25) (layer F.Cu) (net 2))
 (segment (start 91.5 81) (end 90.954177 81) (width 0.25) (layer F.Cu) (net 2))
 (via (at 101.5 84.6) (size 0.8) (drill 0.4) (layers F.Cu B.Cu) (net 2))
 (segment (start 105.81 86.5) (end 107.935001 84.374999) (width 0.25) (layer F.Cu) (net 2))
 (segment (start 107.935001 84.374999) (end 109.875001 84.374999) (width 0.25) (layer F.Cu) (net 2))
 (segment (start 109.875001 84.374999) (end 113.9 80.35) (width 0.25) (layer F.Cu) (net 2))
 (segment (start 113.9 80.35) (end 113.9 78.7) (width 0.25) (layer F.Cu) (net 2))
 (segment (start 87.949988 86.89505) (end 89.30495 86.89505) (width 0.25) (layer B.Cu) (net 3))
 (segment (start 89.30495 86.89505) (end 89.4 86.8) (width 0.25) (layer B.Cu) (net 3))
 (segment (start 87.949988 86.89505) (end 87.264938 86.21) (width 0.25) (layer F.Cu) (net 3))
 (segment (start 87.264938 86.21) (end 83.15 86.21) (width 0.25) (layer F.Cu) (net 3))
 (segment (start 87.949988 86.89505) (end 87.949988 87.460735) (width 0.25) (layer F.Cu) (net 3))
 (segment (start 87.949988 87.460735) (end 88.489253 88) (width 0.25) (layer F.Cu) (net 3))
 (segment (start 88.489253 88) (end 91.1 88) (width 0.25) (layer F.Cu) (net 3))
 (segment (start 106.6 77.5) (end 106.8208 77.2792) (width 0.25) (layer F.Cu) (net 3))
 (segment (start 106.8208 77.2792) (end 107.432 77.2792) (width 0.25) (layer F.Cu) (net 3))
 (segment (start 106.6 78.3482) (end 106.6 77.5) (width 0.25) (layer F.Cu) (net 3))
 (segment (start 107.432 78.6) (end 106.8518 78.6) (width 0.25) (layer F.Cu) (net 3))
 (segment (start 106.8518 78.6) (end 106.6 78.3482) (width 0.25) (layer F.Cu) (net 3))
 (segment (start 91.75 86.4) (end 91.75 87.4) (width 0.25) (layer F.Cu) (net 3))
 (segment (start 91.75 87.4) (end 91.65 87.5) (width 0.25) (layer F.Cu) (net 3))
 (segment (start 107.432 78.6) (end 107.432 79.781002) (width 0.25) (layer F.Cu) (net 3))
 (segment (start 107.432 79.781002) (end 101.736503 85.476499) (width 0.25) (layer F.Cu) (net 3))
 (segment (start 101.736503 85.476499) (end 100.023501 85.476499) (width 0.25) (layer F.Cu) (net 3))
 (segment (start 100.023501 85.476499) (end 99.4 86.1) (width 0.25) (layer F.Cu) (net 3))
 (segment (start 99.4 86.1) (end 99.4 87.5) (width 0.25) (layer F.Cu) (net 3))
 (segment (start 99.4 87.5) (end 98.999977 87.900023) (width 0.25) (layer F.Cu) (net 3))
 (segment (start 98.999977 87.900023) (end 95.899977 87.900023) (width 0.25) (layer F.Cu) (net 3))
 (segment (start 95.899977 87.900023) (end 94.7 87.900023) (width 0.25) (layer F.Cu) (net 3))
 (segment (start 107.432 78.6) (end 108.55 78.6) (width 0.25) (layer F.Cu) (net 3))
 (segment (start 108.55 78.6) (end 108.7 78.45) (width 0.25) (layer F.Cu) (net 3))
 (segment (start 86.2 86.21) (end 83.15 86.21) (width 0.25) (layer F.Cu) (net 3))
 (segment (start 87.4 85.01) (end 86.2 86.21) (width 0.25) (layer F.Cu) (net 3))
 (segment (start 91.7 82.1) (end 90.773004 82.1) (width 0.25) (layer F.Cu) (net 3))
 (segment (start 87.863004 85.01) (end 87.4 85.01) (width 0.25) (layer F.Cu) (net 3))
 (segment (start 90.773004 82.1) (end 87.863004 85.01) (width 0.25) (layer F.Cu) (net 3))
 (segment (start 88.045038 86.8) (end 87.949988 86.89505) (width 0.25) (layer B.Cu) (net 3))
 (via (at 89.4 86.8) (size 0.8) (drill 0.4) (layers F.Cu B.Cu) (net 3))
 (segment (start 94.7 87.900023) (end 88.954961 87.900023) (width 0.25) (layer B.Cu) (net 3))
 (segment (start 91.6 87.5) (end 91.65 87.5) (width 0.25) (layer F.Cu) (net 3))
 (segment (start 91.1 88) (end 91.6 87.5) (width 0.25) (layer F.Cu) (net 3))
 (segment (start 88.954961 87.900023) (end 88.349987 87.295049) (width 0.25) (layer B.Cu) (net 3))
 (via (at 87.949988 86.89505) (size 0.8) (drill 0.4) (layers F.Cu B.Cu) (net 3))
 (segment (start 91.65 85.1) (end 91.1 85.1) (width 0.25) (layer F.Cu) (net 3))
 (segment (start 91.1 85.1) (end 89.4 86.8) (width 0.25) (layer F.Cu) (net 3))
 (segment (start 88.349987 87.295049) (end 87.949988 86.89505) (width 0.25) (layer B.Cu) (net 3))
 (via (at 94.7 87.900023) (size 0.8) (drill 0.4) (layers F.Cu B.Cu) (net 3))
 (segment (start 91.7 82.1) (end 91.5 81.9) (width 0.25) (layer F.Cu) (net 3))
 (segment (start 92.05 82.45) (end 91.7 82.1) (width 0.25) (layer F.Cu) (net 3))
 (segment (start 92.45 82.45) (end 92.05 82.45) (width 0.25) (layer F.Cu) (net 3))
 (segment (start 91.5 81.9) (end 91.5 81.5) (width 0.25) (layer F.Cu) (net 3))
 (segment (start 103.699999 80.04999) (end 103.3 80.449989) (width 0.25) (layer F.Cu) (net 4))
 (segment (start 104.1 79.649989) (end 103.699999 80.04999) (width 0.25) (layer F.Cu) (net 4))
 (segment (start 90.319533 80.449989) (end 102.734315 80.449989) (width 0.25) (layer B.Cu) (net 4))
 (segment (start 102.734315 80.449989) (end 103.3 80.449989) (width 0.25) (layer B.Cu) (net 4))
 (segment (start 88.1 82.669522) (end 90.319533 80.449989) (width 0.25) (layer B.Cu) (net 4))
 (segment (start 104.1 78.4) (end 104.1 79.649989) (width 0.25) (layer F.Cu) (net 4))
 (via (at 103.3 80.449989) (size 0.8) (drill 0.4) (layers F.Cu B.Cu) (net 4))
 (segment (start 105.4 78.6) (end 104.3 78.6) (width 0.25) (layer F.Cu) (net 4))
 (segment (start 104.3 78.6) (end 104.1 78.4) (width 0.25) (layer F.Cu) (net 4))
 (segment (start 88 82.769522) (end 87.868645 82.900877) (width 0.25) (layer F.Cu) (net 4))
 (segment (start 87.868645 82.900877) (end 87.857847 82.900877) (width 0.25) (layer B.Cu) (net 4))
 (via (at 87.857847 82.900877) (size 0.8) (drill 0.4) (layers F.Cu B.Cu) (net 4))
 (segment (start 87.868645 82.900877) (end 87.857847 82.900877) (width 0.25) (layer F.Cu) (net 4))
 (segment (start 88.1 82.669522) (end 87.868645 82.900877) (width 0.25) (layer B.Cu) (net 4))
 (segment (start 88.1 82.669522) (end 87.885681 82.883841) (width 0.25) (layer B.Cu) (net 4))
 (segment (start 91.5 80.5) (end 90.269522 80.5) (width 0.25) (layer F.Cu) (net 4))
 (segment (start 88.28568 82.483842) (end 87.885681 82.883841) (width 0.25) (layer F.Cu) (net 4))
 (segment (start 90.269522 80.5) (end 88.28568 82.483842) (width 0.25) (layer F.Cu) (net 4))
 (segment (start 83.4 81.1) (end 86.15 81.1) (width 0.25) (layer F.Cu) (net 5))
 (segment (start 86.15 81.1) (end 87.75 79.5) (width 0.25) (layer F.Cu) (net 5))
 (segment (start 90.825 79.5) (end 91.5 79.5) (width 0.25) (layer F.Cu) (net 5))
 (segment (start 87.75 79.5) (end 90.825 79.5) (width 0.25) (layer F.Cu) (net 5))
 (segment (start 90.825 80) (end 91.5 80) (width 0.25) (layer F.Cu) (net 6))
 (segment (start 89.710672 80) (end 90.825 80) (width 0.25) (layer F.Cu) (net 6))
 (segment (start 83.4 83.7) (end 86.010672 83.7) (width 0.25) (layer F.Cu) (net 6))
 (segment (start 86.010672 83.7) (end 89.710672 80) (width 0.25) (layer F.Cu) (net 6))
 (segment (start 100.6 83.6) (end 100.6 86.37) (width 0.25) (layer B.Cu) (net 7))
 (segment (start 100.6 86.37) (end 100.73 86.5) (width 0.25) (layer B.Cu) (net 7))
 (segment (start 101.3 81.5) (end 101.3 82.9) (width 0.25) (layer F.Cu) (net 7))
 (segment (start 101.3 82.9) (end 100.6 83.6) (width 0.25) (layer F.Cu) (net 7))
 (via (at 100.6 83.6) (size 0.8) (drill 0.4) (layers F.Cu B.Cu) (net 7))
 (segment (start 94.525 76.8) (end 98.45 76.8) (width 0.25) (layer F.Cu) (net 7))
 (segment (start 98.45 76.8) (end 100.35 78.7) (width 0.25) (layer F.Cu) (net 7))
 (segment (start 100.35 78.7) (end 101.7 78.7) (width 0.25) (layer F.Cu) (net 7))
 (segment (start 94.45 77.55) (end 94.45 76.875) (width 0.25) (layer F.Cu) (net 7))
 (segment (start 94.45 76.875) (end 94.525 76.8) (width 0.25) (layer F.Cu) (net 7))
 (segment (start 101.3 81.5) (end 101.7 81.1) (width 0.25) (layer F.Cu) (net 7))
 (segment (start 101.7 81.1) (end 101.7 78.7) (width 0.25) (layer F.Cu) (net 7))
 (segment (start 109.2 86.1) (end 107.95 86.1) (width 0.25) (layer F.Cu) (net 8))
 (segment (start 107.95 86.1) (end 106.526499 87.523501) (width 0.25) (layer F.Cu) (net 8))
 (segment (start 105.123501 87.523501) (end 104.6 87) (width 0.25) (layer F.Cu) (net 8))
 (segment (start 106.526499 87.523501) (end 105.123501 87.523501) (width 0.25) (layer F.Cu) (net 8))
 (segment (start 104.6 87) (end 104.6 85.2) (width 0.25) (layer F.Cu) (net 8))
 (segment (start 104.6 85.2) (end 106 83.8) (width 0.25) (layer F.Cu) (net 8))
 (segment (start 99.7 81.4) (end 99.7 84.99) (width 0.25) (layer B.Cu) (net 8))
 (segment (start 99.7 84.99) (end 98.19 86.5) (width 0.25) (layer B.Cu) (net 8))
 (segment (start 99.925001 81.174999) (end 99.7 81.4) (width 0.25) (layer B.Cu) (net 8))
 (segment (start 106 83.8) (end 106 83.234315) (width 0.25) (layer B.Cu) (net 8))
 (segment (start 106 83.234315) (end 103.940684 81.174999) (width 0.25) (layer B.Cu) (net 8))
 (segment (start 103.940684 81.174999) (end 99.925001 81.174999) (width 0.25) (layer B.Cu) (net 8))
 (via (at 106 83.8) (size 0.8) (drill 0.4) (layers F.Cu B.Cu) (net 8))
 (segment (start 98.19 79.343235) (end 98.2 79.333235) (width 0.25) (layer F.Cu) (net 8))
 (segment (start 98.2 79.333235) (end 98.2 78.4) (width 0.25) (layer F.Cu) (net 8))
 (segment (start 98.2 77.7) (end 98.2 78.4) (width 0.25) (layer B.Cu) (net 8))
 (via (at 98.2 78.4) (size 0.8) (drill 0.4) (layers F.Cu B.Cu) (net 8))
 (segment (start 97.3 76.8) (end 98.2 77.7) (width 0.25) (layer B.Cu) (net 8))
 (segment (start 91.4 76.8) (end 97.3 76.8) (width 0.25) (layer B.Cu) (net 8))
 (segment (start 91.3 76.9) (end 91.4 76.8) (width 0.25) (layer B.Cu) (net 8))
 (segment (start 93.875 76.8) (end 91.4 76.8) (width 0.25) (layer F.Cu) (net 8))
 (segment (start 91.4 76.8) (end 91.3 76.9) (width 0.25) (layer F.Cu) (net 8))
 (via (at 91.3 76.9) (size 0.8) (drill 0.4) (layers F.Cu B.Cu) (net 8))
 (segment (start 93.95 77.55) (end 93.95 76.875) (width 0.25) (layer F.Cu) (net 8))
 (segment (start 93.95 76.875) (end 93.875 76.8) (width 0.25) (layer F.Cu) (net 8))
 (segment (start 98.19 86.5) (end 98.19 79.343235) (width 0.25) (layer F.Cu) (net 8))
 (segment (start 92.95 82.45) (end 92.95 83.125) (width 0.25) (layer F.Cu) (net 9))
 (segment (start 90.725002 86.974998) (end 90.725002 86.189996) (width 0.25) (layer F.Cu) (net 9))
 (segment (start 92.95 83.125) (end 92.87499 83.20001) (width 0.25) (layer F.Cu) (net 9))
 (segment (start 90.725002 86.189996) (end 91.214998 85.7) (width 0.25) (layer F.Cu) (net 9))
 (segment (start 92.87499 83.20001) (end 90.309405 83.20001) (width 0.25) (layer F.Cu) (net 9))
 (segment (start 91.214998 85.7) (end 92.5 85.7) (width 0.25) (layer F.Cu) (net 9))
 (segment (start 90.309405 83.20001) (end 88.174999 85.334416) (width 0.25) (layer F.Cu) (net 9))
 (segment (start 88.174999 85.334416) (end 88.174999 85.848001) (width 0.25) (layer F.Cu) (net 9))
 (segment (start 88.174999 85.848001) (end 88.674998 86.348) (width 0.25) (layer F.Cu) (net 9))
 (segment (start 88.674998 86.348) (end 88.674998 87.148002) (width 0.25) (layer F.Cu) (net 9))
 (segment (start 88.674998 87.148002) (end 89.051998 87.525002) (width 0.25) (layer F.Cu) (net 9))
 (segment (start 89.051998 87.525002) (end 90.174998 87.525002) (width 0.25) (layer F.Cu) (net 9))
 (segment (start 90.174998 87.525002) (end 90.725002 86.974998) (width 0.25) (layer F.Cu) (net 9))
 (segment (start 92.65 85.85) (end 92.65 86.4) (width 0.25) (layer F.Cu) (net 9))
 (segment (start 92.5 85.7) (end 92.65 85.85) (width 0.25) (layer F.Cu) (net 9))
 (segment (start 92.95 82.45) (end 92.95 82.896765) (width 0.25) (layer F.Cu) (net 9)))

